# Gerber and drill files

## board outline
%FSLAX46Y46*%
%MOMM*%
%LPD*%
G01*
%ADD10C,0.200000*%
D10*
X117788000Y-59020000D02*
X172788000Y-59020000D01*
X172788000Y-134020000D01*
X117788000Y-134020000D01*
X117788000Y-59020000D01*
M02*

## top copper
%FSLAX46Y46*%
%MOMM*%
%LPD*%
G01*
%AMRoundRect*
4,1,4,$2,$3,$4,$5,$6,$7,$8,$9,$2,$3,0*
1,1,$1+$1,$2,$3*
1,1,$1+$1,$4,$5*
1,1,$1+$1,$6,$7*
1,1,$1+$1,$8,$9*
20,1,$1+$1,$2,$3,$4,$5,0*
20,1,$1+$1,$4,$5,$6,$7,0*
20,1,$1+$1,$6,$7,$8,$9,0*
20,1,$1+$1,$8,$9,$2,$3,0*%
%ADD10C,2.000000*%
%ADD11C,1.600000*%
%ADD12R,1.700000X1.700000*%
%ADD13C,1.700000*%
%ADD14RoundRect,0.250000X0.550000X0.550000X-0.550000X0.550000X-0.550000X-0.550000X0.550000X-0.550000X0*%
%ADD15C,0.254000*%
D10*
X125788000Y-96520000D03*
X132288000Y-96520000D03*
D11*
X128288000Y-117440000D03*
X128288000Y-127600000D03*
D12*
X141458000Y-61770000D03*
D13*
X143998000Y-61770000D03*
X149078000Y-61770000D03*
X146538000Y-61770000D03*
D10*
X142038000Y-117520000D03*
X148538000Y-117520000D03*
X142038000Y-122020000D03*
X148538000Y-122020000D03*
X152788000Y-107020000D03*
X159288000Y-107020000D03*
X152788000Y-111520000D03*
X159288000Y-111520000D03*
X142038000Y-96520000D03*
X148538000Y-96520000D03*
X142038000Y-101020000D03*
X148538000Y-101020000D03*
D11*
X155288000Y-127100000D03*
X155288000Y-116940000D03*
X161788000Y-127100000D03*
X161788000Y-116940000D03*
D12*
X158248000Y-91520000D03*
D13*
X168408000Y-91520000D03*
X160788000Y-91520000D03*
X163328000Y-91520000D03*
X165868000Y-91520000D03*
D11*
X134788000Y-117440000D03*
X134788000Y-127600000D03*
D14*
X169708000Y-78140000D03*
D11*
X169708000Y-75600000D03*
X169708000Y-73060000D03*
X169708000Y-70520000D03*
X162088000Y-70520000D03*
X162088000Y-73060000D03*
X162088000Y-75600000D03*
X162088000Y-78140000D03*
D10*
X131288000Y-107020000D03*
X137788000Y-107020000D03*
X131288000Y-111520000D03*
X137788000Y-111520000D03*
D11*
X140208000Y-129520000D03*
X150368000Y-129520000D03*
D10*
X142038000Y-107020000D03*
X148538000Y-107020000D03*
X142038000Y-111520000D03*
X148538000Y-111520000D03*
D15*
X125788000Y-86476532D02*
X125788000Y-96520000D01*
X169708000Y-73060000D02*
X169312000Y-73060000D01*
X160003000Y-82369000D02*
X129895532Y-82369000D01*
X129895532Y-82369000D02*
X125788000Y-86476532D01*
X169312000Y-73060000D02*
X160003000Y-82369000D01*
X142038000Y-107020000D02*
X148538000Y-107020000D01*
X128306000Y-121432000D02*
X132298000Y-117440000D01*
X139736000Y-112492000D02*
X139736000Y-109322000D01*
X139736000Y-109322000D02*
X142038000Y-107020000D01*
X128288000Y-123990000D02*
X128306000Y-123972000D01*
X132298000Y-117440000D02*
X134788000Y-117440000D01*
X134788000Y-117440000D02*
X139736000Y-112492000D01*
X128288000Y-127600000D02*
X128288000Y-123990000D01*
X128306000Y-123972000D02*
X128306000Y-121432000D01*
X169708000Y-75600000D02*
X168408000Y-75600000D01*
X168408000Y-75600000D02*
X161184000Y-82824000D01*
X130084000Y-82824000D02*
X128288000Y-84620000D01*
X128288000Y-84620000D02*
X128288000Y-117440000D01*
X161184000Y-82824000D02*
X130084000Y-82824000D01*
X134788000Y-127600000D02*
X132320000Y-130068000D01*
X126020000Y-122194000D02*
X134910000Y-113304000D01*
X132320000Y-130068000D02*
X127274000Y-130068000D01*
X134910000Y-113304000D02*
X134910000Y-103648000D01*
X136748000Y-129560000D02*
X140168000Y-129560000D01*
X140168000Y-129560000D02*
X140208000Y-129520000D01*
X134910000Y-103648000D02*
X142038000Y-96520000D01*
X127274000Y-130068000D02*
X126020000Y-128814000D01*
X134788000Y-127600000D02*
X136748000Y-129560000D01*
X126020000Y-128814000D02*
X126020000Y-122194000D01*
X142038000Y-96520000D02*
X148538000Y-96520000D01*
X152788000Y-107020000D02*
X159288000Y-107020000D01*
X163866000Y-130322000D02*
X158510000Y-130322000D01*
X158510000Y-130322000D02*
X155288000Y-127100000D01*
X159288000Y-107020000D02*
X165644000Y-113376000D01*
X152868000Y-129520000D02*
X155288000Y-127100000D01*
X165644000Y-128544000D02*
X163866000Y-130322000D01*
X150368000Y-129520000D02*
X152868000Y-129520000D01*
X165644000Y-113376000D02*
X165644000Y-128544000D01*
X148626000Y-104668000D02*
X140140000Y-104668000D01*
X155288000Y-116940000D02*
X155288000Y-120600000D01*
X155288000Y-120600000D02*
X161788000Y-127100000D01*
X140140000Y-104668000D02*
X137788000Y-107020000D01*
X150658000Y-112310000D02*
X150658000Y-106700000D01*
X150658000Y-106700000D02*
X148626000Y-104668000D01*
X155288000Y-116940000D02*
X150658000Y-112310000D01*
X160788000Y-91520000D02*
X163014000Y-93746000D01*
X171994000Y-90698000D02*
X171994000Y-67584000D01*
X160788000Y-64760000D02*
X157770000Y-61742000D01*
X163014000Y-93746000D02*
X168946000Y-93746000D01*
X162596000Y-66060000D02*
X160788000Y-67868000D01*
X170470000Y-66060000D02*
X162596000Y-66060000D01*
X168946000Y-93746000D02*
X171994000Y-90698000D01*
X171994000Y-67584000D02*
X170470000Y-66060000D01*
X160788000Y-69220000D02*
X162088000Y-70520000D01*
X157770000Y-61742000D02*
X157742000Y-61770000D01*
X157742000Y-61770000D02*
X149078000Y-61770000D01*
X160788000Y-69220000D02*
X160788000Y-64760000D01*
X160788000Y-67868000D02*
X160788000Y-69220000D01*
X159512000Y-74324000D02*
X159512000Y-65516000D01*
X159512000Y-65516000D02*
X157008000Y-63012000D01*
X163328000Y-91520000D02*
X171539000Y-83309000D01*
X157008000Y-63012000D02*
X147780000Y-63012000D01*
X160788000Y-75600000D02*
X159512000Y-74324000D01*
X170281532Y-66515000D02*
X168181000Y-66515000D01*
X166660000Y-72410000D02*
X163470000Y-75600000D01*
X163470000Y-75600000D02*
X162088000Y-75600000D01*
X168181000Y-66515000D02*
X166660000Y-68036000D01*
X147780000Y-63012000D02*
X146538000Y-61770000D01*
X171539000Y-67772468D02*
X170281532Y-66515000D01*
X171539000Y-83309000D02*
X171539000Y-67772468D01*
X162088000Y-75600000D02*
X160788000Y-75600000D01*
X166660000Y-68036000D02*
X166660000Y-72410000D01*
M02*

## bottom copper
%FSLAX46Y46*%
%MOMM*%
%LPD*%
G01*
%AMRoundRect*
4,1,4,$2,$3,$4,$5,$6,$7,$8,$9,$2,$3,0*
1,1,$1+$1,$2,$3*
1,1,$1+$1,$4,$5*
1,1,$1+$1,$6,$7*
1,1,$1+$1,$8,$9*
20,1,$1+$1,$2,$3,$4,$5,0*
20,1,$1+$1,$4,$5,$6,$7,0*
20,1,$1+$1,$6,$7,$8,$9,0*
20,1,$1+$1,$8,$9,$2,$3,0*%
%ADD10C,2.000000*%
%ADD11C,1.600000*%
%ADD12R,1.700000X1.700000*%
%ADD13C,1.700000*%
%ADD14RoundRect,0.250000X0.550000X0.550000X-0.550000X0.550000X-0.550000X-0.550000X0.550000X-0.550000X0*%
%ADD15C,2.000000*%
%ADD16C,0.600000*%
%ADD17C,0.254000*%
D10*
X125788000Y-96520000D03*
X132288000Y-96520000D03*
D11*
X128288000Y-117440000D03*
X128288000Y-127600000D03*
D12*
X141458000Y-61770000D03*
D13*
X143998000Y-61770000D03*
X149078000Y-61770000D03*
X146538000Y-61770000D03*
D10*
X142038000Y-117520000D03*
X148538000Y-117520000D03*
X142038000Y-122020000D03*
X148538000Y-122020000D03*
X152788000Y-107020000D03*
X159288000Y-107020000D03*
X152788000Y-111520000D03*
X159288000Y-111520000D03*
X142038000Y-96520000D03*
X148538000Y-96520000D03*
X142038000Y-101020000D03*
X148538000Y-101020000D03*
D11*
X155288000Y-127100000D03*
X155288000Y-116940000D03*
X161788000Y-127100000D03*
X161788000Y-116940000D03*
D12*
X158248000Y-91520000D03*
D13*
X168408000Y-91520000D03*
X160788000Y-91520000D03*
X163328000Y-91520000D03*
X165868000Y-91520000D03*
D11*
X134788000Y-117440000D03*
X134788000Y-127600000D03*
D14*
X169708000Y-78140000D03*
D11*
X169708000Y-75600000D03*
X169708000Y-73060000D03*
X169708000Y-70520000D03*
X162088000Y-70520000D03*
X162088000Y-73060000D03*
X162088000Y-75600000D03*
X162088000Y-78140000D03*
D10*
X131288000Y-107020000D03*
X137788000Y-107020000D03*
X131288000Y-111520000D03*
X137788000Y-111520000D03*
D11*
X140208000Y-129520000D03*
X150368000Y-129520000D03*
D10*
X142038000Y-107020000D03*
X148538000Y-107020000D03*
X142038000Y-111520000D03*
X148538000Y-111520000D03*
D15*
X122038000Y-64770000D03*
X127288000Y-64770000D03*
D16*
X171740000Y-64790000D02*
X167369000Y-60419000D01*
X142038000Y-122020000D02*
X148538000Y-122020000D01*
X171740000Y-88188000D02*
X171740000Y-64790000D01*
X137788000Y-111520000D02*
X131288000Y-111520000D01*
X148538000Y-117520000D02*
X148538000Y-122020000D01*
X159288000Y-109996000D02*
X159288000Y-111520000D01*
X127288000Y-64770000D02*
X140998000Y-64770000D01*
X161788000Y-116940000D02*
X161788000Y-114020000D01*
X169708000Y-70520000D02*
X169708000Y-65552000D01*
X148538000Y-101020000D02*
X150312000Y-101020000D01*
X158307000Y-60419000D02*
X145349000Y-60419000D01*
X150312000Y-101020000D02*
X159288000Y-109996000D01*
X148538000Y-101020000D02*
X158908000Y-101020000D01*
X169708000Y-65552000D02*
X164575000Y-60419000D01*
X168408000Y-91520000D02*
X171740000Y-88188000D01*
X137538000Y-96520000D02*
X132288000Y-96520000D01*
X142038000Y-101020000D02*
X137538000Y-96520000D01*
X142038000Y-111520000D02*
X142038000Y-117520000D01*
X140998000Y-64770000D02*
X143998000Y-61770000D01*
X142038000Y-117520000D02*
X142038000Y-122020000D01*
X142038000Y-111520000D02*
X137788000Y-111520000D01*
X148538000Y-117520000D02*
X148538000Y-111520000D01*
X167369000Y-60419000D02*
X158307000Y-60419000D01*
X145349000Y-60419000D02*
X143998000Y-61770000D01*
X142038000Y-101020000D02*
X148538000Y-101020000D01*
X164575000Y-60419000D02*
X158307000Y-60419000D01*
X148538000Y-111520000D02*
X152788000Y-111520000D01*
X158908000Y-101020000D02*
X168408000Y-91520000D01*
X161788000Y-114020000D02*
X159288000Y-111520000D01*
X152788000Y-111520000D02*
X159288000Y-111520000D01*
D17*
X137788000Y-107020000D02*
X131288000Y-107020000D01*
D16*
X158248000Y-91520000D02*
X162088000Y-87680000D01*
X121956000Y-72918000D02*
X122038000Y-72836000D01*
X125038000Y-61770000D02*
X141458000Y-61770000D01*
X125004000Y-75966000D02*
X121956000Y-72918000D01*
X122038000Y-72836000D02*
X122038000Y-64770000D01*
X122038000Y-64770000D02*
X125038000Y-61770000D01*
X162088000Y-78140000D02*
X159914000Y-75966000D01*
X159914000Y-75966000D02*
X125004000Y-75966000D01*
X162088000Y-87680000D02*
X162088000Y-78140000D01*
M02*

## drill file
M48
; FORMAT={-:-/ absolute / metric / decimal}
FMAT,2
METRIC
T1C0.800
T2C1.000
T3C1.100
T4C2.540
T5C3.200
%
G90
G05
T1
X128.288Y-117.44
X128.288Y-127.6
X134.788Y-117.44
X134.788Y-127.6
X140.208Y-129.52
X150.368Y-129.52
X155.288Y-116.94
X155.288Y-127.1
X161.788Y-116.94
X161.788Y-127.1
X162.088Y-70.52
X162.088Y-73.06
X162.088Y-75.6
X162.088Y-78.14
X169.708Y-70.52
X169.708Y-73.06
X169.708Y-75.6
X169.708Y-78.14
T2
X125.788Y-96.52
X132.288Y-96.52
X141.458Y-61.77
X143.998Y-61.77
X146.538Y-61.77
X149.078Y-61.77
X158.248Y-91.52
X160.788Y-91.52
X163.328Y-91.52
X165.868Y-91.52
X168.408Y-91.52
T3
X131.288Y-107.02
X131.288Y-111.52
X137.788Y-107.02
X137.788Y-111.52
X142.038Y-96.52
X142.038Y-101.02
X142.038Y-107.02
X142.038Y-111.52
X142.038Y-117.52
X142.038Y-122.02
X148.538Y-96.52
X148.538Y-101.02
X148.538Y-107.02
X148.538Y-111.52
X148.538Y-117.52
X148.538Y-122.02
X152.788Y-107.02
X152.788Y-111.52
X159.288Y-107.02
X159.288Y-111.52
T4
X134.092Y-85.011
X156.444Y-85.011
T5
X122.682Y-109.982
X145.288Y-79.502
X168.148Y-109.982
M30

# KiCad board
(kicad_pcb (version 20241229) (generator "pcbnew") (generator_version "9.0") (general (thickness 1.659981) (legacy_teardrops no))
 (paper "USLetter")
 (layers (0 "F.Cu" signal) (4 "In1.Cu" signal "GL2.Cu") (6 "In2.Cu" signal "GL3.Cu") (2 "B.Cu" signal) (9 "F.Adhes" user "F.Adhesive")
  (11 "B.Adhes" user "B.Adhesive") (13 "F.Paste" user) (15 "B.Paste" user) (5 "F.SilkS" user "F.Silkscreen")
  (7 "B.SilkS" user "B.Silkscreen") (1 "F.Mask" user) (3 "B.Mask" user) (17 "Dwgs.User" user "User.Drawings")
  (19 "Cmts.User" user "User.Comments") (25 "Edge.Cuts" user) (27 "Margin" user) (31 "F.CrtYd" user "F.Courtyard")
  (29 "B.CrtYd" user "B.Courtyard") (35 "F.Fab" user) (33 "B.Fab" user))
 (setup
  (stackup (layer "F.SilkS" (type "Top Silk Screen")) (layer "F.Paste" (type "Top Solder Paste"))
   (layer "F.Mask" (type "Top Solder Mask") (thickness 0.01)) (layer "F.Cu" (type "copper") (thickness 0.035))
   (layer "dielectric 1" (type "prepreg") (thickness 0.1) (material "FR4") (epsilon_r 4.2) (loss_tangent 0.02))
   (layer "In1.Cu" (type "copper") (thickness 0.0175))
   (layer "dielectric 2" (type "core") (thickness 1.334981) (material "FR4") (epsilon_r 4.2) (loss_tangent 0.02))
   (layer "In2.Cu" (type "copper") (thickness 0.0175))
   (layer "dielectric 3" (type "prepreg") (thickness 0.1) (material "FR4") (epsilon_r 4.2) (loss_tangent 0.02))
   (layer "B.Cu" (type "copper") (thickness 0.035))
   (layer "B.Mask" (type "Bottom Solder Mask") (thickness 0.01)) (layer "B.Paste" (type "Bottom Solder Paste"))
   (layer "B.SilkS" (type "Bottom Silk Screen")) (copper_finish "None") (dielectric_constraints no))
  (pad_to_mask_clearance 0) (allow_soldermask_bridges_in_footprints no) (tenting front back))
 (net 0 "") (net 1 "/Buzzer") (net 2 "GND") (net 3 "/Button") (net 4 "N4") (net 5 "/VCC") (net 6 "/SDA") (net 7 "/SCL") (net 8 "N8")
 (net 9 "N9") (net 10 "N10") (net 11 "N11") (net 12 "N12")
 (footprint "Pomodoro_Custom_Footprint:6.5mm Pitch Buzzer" (layer "F.Cu") (at 129.038 96.52)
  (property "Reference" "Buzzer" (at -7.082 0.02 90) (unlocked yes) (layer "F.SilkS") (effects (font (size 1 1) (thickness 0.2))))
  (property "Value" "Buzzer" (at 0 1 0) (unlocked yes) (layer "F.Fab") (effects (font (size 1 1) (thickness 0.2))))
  (pad "1" thru_hole circle (at -3.25 0) (size 2 2) (drill 1) (layers "*.Cu" "*.Mask") (remove_unused_layers no) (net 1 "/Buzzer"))
  (pad "2" thru_hole circle (at 3.25 0) (size 2 2) (drill 1) (layers "*.Cu" "*.Mask") (remove_unused_layers no) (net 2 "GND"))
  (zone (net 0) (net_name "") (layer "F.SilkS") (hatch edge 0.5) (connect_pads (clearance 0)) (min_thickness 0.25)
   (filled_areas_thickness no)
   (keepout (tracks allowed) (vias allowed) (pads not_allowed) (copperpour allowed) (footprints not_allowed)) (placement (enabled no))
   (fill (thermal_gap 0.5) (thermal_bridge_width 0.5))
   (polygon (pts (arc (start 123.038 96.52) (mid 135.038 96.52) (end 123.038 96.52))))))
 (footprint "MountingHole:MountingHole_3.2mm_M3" (layer "F.Cu") (at 168.148 109.982)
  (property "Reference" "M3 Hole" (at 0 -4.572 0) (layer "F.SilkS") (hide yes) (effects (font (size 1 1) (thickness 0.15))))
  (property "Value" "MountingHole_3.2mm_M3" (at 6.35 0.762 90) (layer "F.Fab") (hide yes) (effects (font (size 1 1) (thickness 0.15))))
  (pad "" np_thru_hole circle (at 0 0) (size 3.2 3.2) (drill 3.2) (layers "*.Cu" "*.Mask")))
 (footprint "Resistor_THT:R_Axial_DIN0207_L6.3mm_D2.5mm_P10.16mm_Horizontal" (layer "F.Cu") (at 128.288 117.44 -90)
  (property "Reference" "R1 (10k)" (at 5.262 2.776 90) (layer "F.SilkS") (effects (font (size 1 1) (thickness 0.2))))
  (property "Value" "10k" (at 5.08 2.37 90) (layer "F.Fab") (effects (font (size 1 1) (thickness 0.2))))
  (pad "1" thru_hole circle (at 0 0 270) (size 1.6 1.6) (drill 0.8) (layers "*.Cu" "*.Mask") (remove_unused_layers no) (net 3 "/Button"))
  (pad "2" thru_hole circle (at 10.16 0 270) (size 1.6 1.6) (drill 0.8) (layers "*.Cu" "*.Mask") (remove_unused_layers no) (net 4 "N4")))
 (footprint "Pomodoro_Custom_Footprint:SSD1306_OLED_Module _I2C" (layer "F.Cu") (at 145.268 73.835)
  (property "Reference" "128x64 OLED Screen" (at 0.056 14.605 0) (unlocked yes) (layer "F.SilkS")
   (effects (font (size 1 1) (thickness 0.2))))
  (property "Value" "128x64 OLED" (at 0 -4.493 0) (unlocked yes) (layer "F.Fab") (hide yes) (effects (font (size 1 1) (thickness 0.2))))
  (pad "" np_thru_hole circle (at -11.176 11.176) (size 1.7 1.7) (drill 2.54) (layers "*.Cu" "*.Mask"))
  (pad "" np_thru_hole circle (at 11.176 11.176) (size 1.7 1.7) (drill 2.54) (layers "*.Cu" "*.Mask"))
  (pad "1" thru_hole rect (at -3.81 -12.065) (size 1.7 1.7) (drill 1) (layers "*.Cu" "*.Mask") (remove_unused_layers no) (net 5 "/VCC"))
  (pad "2" thru_hole circle (at -1.27 -12.065) (size 1.7 1.7) (drill 1) (layers "*.Cu" "*.Mask") (remove_unused_layers no) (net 2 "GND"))
  (pad "3" thru_hole circle (at 3.81 -12.065) (size 1.7 1.7) (drill 1) (layers "*.Cu" "*.Mask") (remove_unused_layers no) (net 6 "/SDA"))
  (pad "4" thru_hole circle (at 1.27 -12.065) (size 1.7 1.7) (drill 1) (layers "*.Cu" "*.Mask") (remove_unused_layers no) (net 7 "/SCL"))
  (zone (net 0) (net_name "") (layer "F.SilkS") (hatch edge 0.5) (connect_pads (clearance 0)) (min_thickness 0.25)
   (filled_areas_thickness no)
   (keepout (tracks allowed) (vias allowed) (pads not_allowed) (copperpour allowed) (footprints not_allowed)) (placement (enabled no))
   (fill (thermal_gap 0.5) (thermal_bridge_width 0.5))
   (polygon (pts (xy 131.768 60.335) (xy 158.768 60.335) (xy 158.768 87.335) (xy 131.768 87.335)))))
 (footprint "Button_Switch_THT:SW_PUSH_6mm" (layer "F.Cu") (at 142.038 117.52)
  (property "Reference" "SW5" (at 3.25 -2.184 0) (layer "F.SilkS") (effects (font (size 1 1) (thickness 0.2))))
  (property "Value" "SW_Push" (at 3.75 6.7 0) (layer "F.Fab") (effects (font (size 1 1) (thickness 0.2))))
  (pad "1" thru_hole circle (at 0 0 90) (size 2 2) (drill 1.1) (layers "*.Cu" "*.Mask") (remove_unused_layers no) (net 2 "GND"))
  (pad "1" thru_hole circle (at 6.5 0 90) (size 2 2) (drill 1.1) (layers "*.Cu" "*.Mask") (remove_unused_layers no) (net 2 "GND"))
  (pad "2" thru_hole circle (at 0 4.5 90) (size 2 2) (drill 1.1) (layers "*.Cu" "*.Mask") (remove_unused_layers no) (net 2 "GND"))
  (pad "2" thru_hole circle (at 6.5 4.5 90) (size 2 2) (drill 1.1) (layers "*.Cu" "*.Mask") (remove_unused_layers no) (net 2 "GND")))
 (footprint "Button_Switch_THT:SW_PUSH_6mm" (layer "F.Cu") (at 152.788 107.02)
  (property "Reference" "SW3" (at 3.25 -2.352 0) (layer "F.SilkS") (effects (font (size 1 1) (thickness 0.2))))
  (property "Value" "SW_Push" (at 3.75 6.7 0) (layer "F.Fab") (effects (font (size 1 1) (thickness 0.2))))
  (pad "1" thru_hole circle (at 0 0 90) (size 2 2) (drill 1.1) (layers "*.Cu" "*.Mask") (remove_unused_layers no) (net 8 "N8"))
  (pad "1" thru_hole circle (at 6.5 0 90) (size 2 2) (drill 1.1) (layers "*.Cu" "*.Mask") (remove_unused_layers no) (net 8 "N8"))
  (pad "2" thru_hole circle (at 0 4.5 90) (size 2 2) (drill 1.1) (layers "*.Cu" "*.Mask") (remove_unused_layers no) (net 2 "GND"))
  (pad "2" thru_hole circle (at 6.5 4.5 90) (size 2 2) (drill 1.1) (layers "*.Cu" "*.Mask") (remove_unused_layers no) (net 2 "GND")))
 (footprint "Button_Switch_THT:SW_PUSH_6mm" (layer "F.Cu") (at 142.038 96.52)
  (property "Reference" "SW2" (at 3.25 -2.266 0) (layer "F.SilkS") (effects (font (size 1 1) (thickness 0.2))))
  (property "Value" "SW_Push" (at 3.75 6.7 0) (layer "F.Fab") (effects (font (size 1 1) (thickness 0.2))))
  (pad "1" thru_hole circle (at 0 0 90) (size 2 2) (drill 1.1) (layers "*.Cu" "*.Mask") (remove_unused_layers no) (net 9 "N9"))
  (pad "1" thru_hole circle (at 6.5 0 90) (size 2 2) (drill 1.1) (layers "*.Cu" "*.Mask") (remove_unused_layers no) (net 9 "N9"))
  (pad "2" thru_hole circle (at 0 4.5 90) (size 2 2) (drill 1.1) (layers "*.Cu" "*.Mask") (remove_unused_layers no) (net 2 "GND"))
  (pad "2" thru_hole circle (at 6.5 4.5 90) (size 2 2) (drill 1.1) (layers "*.Cu" "*.Mask") (remove_unused_layers no) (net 2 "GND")))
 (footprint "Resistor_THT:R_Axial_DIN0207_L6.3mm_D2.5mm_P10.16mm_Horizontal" (layer "F.Cu") (at 155.288 127.1 90)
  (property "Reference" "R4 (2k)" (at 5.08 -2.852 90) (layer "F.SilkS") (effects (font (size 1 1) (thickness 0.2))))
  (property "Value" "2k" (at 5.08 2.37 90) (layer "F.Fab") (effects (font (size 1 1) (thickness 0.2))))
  (pad "1" thru_hole circle (at 0 0 90) (size 1.6 1.6) (drill 0.8) (layers "*.Cu" "*.Mask") (remove_unused_layers no) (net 8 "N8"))
  (pad "2" thru_hole circle (at 10.16 0 90) (size 1.6 1.6) (drill 0.8) (layers "*.Cu" "*.Mask") (remove_unused_layers no) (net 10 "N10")))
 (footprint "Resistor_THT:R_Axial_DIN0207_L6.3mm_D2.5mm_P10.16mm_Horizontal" (layer "F.Cu") (at 161.788 127.1 90)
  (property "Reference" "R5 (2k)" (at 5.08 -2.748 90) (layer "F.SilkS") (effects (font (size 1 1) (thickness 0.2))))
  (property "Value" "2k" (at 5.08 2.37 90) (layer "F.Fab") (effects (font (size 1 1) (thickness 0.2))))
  (pad "1" thru_hole circle (at 0 0 90) (size 1.6 1.6) (drill 0.8) (layers "*.Cu" "*.Mask") (remove_unused_layers no) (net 10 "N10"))
  (pad "2" thru_hole circle (at 10.16 0 90) (size 1.6 1.6) (drill 0.8) (layers "*.Cu" "*.Mask") (remove_unused_layers no) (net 2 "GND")))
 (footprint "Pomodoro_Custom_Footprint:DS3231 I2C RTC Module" (layer "F.Cu") (at 163.328 96.6)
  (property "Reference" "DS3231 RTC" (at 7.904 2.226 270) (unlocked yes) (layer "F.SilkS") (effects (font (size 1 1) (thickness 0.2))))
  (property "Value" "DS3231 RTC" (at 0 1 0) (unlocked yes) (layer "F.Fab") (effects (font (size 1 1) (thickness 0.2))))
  (pad "1" thru_hole rect (at -5.08 -5.08) (size 1.7 1.7) (drill 1) (layers "*.Cu" "*.Mask") (remove_unused_layers no) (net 5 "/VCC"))
  (pad "2" thru_hole circle (at 5.08 -5.08) (size 1.7 1.7) (drill 1) (layers "*.Cu" "*.Mask") (remove_unused_layers no) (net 2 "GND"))
  (pad "3" thru_hole circle (at -2.54 -5.08) (size 1.7 1.7) (drill 1) (layers "*.Cu" "*.Mask") (remove_unused_layers no) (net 6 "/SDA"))
  (pad "4" thru_hole circle (at 0 -5.08) (size 1.7 1.7) (drill 1) (layers "*.Cu" "*.Mask") (remove_unused_layers no) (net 7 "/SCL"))
  (pad "5" thru_hole circle (at 2.54 -5.08) (size 1.7 1.7) (drill 1) (layers "*.Cu" "*.Mask") (remove_unused_layers no))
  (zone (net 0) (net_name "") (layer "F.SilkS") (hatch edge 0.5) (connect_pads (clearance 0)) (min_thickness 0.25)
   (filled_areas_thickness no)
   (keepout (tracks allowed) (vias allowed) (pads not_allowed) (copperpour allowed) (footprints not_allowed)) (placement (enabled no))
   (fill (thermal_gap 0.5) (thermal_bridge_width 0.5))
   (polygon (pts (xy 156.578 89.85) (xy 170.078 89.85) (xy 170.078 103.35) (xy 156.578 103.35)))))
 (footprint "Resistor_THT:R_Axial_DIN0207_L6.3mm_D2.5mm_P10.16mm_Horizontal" (layer "F.Cu") (at 134.788 117.44 -90)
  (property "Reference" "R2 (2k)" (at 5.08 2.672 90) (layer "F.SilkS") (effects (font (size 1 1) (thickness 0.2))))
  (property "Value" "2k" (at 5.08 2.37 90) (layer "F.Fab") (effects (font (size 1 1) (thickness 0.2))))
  (pad "1" thru_hole circle (at 0 0 270) (size 1.6 1.6) (drill 0.8) (layers "*.Cu" "*.Mask") (remove_unused_layers no) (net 4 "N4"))
  (pad "2" thru_hole circle (at 10.16 0 270) (size 1.6 1.6) (drill 0.8) (layers "*.Cu" "*.Mask") (remove_unused_layers no) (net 9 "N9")))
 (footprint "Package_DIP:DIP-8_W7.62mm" (layer "F.Cu") (at 169.708 78.14 180)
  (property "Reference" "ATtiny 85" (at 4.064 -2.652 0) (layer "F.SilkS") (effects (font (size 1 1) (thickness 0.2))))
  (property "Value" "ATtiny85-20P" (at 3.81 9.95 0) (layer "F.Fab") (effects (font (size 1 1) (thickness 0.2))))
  (pad "1" thru_hole roundrect (at 0 0 180) (size 1.6 1.6) (drill 0.8) (layers "*.Cu" "*.Mask") (remove_unused_layers no)
   (roundrect_rratio 0.15625) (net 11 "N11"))
  (pad "2" thru_hole circle (at 0 2.54 180) (size 1.6 1.6) (drill 0.8) (layers "*.Cu" "*.Mask") (remove_unused_layers no) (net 3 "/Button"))
  (pad "3" thru_hole circle (at 0 5.08 180) (size 1.6 1.6) (drill 0.8) (layers "*.Cu" "*.Mask") (remove_unused_layers no) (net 1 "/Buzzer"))
  (pad "4" thru_hole circle (at 0 7.62 180) (size 1.6 1.6) (drill 0.8) (layers "*.Cu" "*.Mask") (remove_unused_layers no) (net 2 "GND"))
  (pad "5" thru_hole circle (at 7.62 7.62 180) (size 1.6 1.6) (drill 0.8) (layers "*.Cu" "*.Mask") (remove_unused_layers no) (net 6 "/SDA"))
  (pad "6" thru_hole circle (at 7.62 5.08 180) (size 1.6 1.6) (drill 0.8) (layers "*.Cu" "*.Mask") (remove_unused_layers no) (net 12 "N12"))
  (pad "7" thru_hole circle (at 7.62 2.54 180) (size 1.6 1.6) (drill 0.8) (layers "*.Cu" "*.Mask") (remove_unused_layers no) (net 7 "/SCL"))
  (pad "8" thru_hole circle (at 7.62 0 180) (size 1.6 1.6) (drill 0.8) (layers "*.Cu" "*.Mask") (remove_unused_layers no) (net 5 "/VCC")))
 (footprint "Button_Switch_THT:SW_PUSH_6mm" (layer "F.Cu") (at 131.288 107.02)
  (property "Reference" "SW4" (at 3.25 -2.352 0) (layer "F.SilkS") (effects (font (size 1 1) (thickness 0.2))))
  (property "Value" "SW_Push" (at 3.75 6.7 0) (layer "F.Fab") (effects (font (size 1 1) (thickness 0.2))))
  (pad "1" thru_hole circle (at 0 0 90) (size 2 2) (drill 1.1) (layers "*.Cu" "*.Mask") (remove_unused_layers no) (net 10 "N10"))
  (pad "1" thru_hole circle (at 6.5 0 90) (size 2 2) (drill 1.1) (layers "*.Cu" "*.Mask") (remove_unused_layers no) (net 10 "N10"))
  (pad "2" thru_hole circle (at 0 4.5 90) (size 2 2) (drill 1.1) (layers "*.Cu" "*.Mask") (remove_unused_layers no) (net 2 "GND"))
  (pad "2" thru_hole circle (at 6.5 4.5 90) (size 2 2) (drill 1.1) (layers "*.Cu" "*.Mask") (remove_unused_layers no) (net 2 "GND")))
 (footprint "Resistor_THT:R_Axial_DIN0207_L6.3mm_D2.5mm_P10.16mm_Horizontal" (layer "F.Cu") (at 140.208 129.52)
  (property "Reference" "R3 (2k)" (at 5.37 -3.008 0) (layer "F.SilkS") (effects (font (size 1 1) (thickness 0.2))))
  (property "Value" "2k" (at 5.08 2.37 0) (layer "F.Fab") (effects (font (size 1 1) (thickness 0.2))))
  (pad "1" thru_hole circle (at 0 0) (size 1.6 1.6) (drill 0.8) (layers "*.Cu" "*.Mask") (remove_unused_layers no) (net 9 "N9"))
  (pad "2" thru_hole circle (at 10.16 0) (size 1.6 1.6) (drill 0.8) (layers "*.Cu" "*.Mask") (remove_unused_layers no) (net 8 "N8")))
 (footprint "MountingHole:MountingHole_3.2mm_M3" (layer "F.Cu") (at 145.288 79.502)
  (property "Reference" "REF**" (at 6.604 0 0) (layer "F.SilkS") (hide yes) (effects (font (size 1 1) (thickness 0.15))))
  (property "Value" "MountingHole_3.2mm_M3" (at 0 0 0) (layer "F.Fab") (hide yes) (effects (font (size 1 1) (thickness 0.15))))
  (pad "" np_thru_hole circle (at 0 0) (size 3.2 3.2) (drill 3.2) (layers "*.Cu" "*.Mask")))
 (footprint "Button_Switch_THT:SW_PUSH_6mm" (layer "F.Cu") (at 142.038 107.02)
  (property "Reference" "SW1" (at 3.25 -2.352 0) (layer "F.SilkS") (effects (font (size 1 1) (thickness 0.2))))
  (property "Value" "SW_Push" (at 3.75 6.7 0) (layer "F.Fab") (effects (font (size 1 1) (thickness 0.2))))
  (pad "1" thru_hole circle (at 0 0 90) (size 2 2) (drill 1.1) (layers "*.Cu" "*.Mask") (remove_unused_layers no) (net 4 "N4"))
  (pad "1" thru_hole circle (at 6.5 0 90) (size 2 2) (drill 1.1) (layers "*.Cu" "*.Mask") (remove_unused_layers no) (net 4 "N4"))
  (pad "2" thru_hole circle (at 0 4.5 90) (size 2 2) (drill 1.1) (layers "*.Cu" "*.Mask") (remove_unused_layers no) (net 2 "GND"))
  (pad "2" thru_hole circle (at 6.5 4.5 90) (size 2 2) (drill 1.1) (layers "*.Cu" "*.Mask") (remove_unused_layers no) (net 2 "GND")))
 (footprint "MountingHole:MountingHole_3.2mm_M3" (layer "F.Cu") (at 122.682 109.982)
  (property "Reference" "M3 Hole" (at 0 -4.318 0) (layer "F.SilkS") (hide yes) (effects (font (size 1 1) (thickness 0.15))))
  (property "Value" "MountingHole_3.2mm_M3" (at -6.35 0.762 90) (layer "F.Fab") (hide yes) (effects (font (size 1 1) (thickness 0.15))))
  (pad "" np_thru_hole circle (at 0 0) (size 3.2 3.2) (drill 3.2) (layers "*.Cu" "*.Mask")))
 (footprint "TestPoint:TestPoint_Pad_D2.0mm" (layer "B.Cu") (at 122.038 64.77 180)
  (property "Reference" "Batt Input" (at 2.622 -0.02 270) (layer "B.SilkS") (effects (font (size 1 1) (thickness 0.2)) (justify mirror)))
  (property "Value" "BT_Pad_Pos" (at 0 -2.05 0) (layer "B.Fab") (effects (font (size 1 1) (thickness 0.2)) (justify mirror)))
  (pad "1" smd circle (at 0 0 180) (size 2 2) (layers "B.Cu" "B.Mask") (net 5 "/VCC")))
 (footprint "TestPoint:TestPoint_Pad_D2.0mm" (layer "B.Cu") (at 127.288 64.77 180)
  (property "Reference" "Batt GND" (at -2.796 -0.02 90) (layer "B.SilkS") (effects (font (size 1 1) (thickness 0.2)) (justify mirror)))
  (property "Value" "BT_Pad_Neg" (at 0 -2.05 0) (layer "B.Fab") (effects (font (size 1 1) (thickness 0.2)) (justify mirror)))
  (pad "1" smd circle (at 0 0 180) (size 2 2) (layers "B.Cu" "B.Mask") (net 2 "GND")))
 (gr_rect (start 117.788 59.02) (end 172.788 134.02) (stroke (width 0.2) (type default)) (fill no) (layer "Edge.Cuts"))
 (segment (start 125.788 86.476532) (end 125.788 96.52) (width 0.254) (layer "F.Cu") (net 1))
 (segment (start 169.708 73.06) (end 169.312 73.06) (width 0.254) (layer "F.Cu") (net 1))
 (segment (start 160.003 82.369) (end 129.895532 82.369) (width 0.254) (layer "F.Cu") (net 1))
 (segment (start 129.895532 82.369) (end 125.788 86.476532) (width 0.254) (layer "F.Cu") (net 1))
 (segment (start 169.312 73.06) (end 160.003 82.369) (width 0.254) (layer "F.Cu") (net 1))
 (segment (start 171.74 64.79) (end 167.369 60.419) (width 0.6) (layer "B.Cu") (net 2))
 (segment (start 142.038 122.02) (end 148.538 122.02) (width 0.6) (layer "B.Cu") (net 2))
 (segment (start 171.74 88.188) (end 171.74 64.79) (width 0.6) (layer "B.Cu") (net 2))
 (segment (start 137.788 111.52) (end 131.288 111.52) (width 0.6) (layer "B.Cu") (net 2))
 (segment (start 148.538 117.52) (end 148.538 122.02) (width 0.6) (layer "B.Cu") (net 2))
 (segment (start 159.288 109.996) (end 159.288 111.52) (width 0.6) (layer "B.Cu") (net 2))
 (segment (start 127.288 64.77) (end 140.998 64.77) (width 0.6) (layer "B.Cu") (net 2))
 (segment (start 161.788 116.94) (end 161.788 114.02) (width 0.6) (layer "B.Cu") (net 2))
 (segment (start 169.708 70.52) (end 169.708 65.552) (width 0.6) (layer "B.Cu") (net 2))
 (segment (start 148.538 101.02) (end 150.312 101.02) (width 0.6) (layer "B.Cu") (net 2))
 (segment (start 158.307 60.419) (end 145.349 60.419) (width 0.6) (layer "B.Cu") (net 2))
 (segment (start 150.312 101.02) (end 159.288 109.996) (width 0.6) (layer "B.Cu") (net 2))
 (segment (start 148.538 101.02) (end 158.908 101.02) (width 0.6) (layer "B.Cu") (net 2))
 (segment (start 169.708 65.552) (end 164.575 60.419) (width 0.6) (layer "B.Cu") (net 2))
 (segment (start 168.408 91.52) (end 171.74 88.188) (width 0.6) (layer "B.Cu") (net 2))
 (segment (start 137.538 96.52) (end 132.288 96.52) (width 0.6) (layer "B.Cu") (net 2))
 (segment (start 142.038 101.02) (end 137.538 96.52) (width 0.6) (layer "B.Cu") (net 2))
 (segment (start 142.038 111.52) (end 142.038 117.52) (width 0.6) (layer "B.Cu") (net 2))
 (segment (start 140.998 64.77) (end 143.998 61.77) (width 0.6) (layer "B.Cu") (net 2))
 (segment (start 142.038 117.52) (end 142.038 122.02) (width 0.6) (layer "B.Cu") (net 2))
 (segment (start 142.038 111.52) (end 137.788 111.52) (width 0.6) (layer "B.Cu") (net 2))
 (segment (start 148.538 117.52) (end 148.538 111.52) (width 0.6) (layer "B.Cu") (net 2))
 (segment (start 167.369 60.419) (end 158.307 60.419) (width 0.6) (layer "B.Cu") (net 2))
 (segment (start 145.349 60.419) (end 143.998 61.77) (width 0.6) (layer "B.Cu") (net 2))
 (segment (start 142.038 101.02) (end 148.538 101.02) (width 0.6) (layer "B.Cu") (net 2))
 (segment (start 164.575 60.419) (end 158.307 60.419) (width 0.6) (layer "B.Cu") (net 2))
 (segment (start 148.538 111.52) (end 152.788 111.52) (width 0.6) (layer "B.Cu") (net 2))
 (segment (start 158.908 101.02) (end 168.408 91.52) (width 0.6) (layer "B.Cu") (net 2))
 (segment (start 161.788 114.02) (end 159.288 111.52) (width 0.6) (layer "B.Cu") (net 2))
 (segment (start 152.788 111.52) (end 159.288 111.52) (width 0.6) (layer "B.Cu") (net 2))
 (segment (start 142.038 107.02) (end 148.538 107.02) (width 0.254) (layer "F.Cu") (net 4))
 (segment (start 128.306 121.432) (end 132.298 117.44) (width 0.254) (layer "F.Cu") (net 4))
 (segment (start 139.736 112.492) (end 139.736 109.322) (width 0.254) (layer "F.Cu") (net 4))
 (segment (start 139.736 109.322) (end 142.038 107.02) (width 0.254) (layer "F.Cu") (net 4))
 (segment (start 128.288 123.99) (end 128.306 123.972) (width 0.254) (layer "F.Cu") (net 4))
 (segment (start 132.298 117.44) (end 134.788 117.44) (width 0.254) (layer "F.Cu") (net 4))
 (segment (start 134.788 117.44) (end 139.736 112.492) (width 0.254) (layer "F.Cu") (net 4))
 (segment (start 128.288 127.6) (end 128.288 123.99) (width 0.254) (layer "F.Cu") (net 4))
 (segment (start 128.306 123.972) (end 128.306 121.432) (width 0.254) (layer "F.Cu") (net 4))
 (segment (start 169.708 75.6) (end 168.408 75.6) (width 0.254) (layer "F.Cu") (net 3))
 (segment (start 168.408 75.6) (end 161.184 82.824) (width 0.254) (layer "F.Cu") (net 3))
 (segment (start 130.084 82.824) (end 128.288 84.62) (width 0.254) (layer "F.Cu") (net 3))
 (segment (start 128.288 84.62) (end 128.288 117.44) (width 0.254) (layer "F.Cu") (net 3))
 (segment (start 161.184 82.824) (end 130.084 82.824) (width 0.254) (layer "F.Cu") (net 3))
 (segment (start 134.788 127.6) (end 132.32 130.068) (width 0.254) (layer "F.Cu") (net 9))
 (segment (start 126.02 122.194) (end 134.91 113.304) (width 0.254) (layer "F.Cu") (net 9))
 (segment (start 132.32 130.068) (end 127.274 130.068) (width 0.254) (layer "F.Cu") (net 9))
 (segment (start 134.91 113.304) (end 134.91 103.648) (width 0.254) (layer "F.Cu") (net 9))
 (segment (start 136.748 129.56) (end 140.168 129.56) (width 0.254) (layer "F.Cu") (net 9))
 (segment (start 140.168 129.56) (end 140.208 129.52) (width 0.254) (layer "F.Cu") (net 9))
 (segment (start 134.91 103.648) (end 142.038 96.52) (width 0.254) (layer "F.Cu") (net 9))
 (segment (start 127.274 130.068) (end 126.02 128.814) (width 0.254) (layer "F.Cu") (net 9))
 (segment (start 134.788 127.6) (end 136.748 129.56) (width 0.254) (layer "F.Cu") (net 9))
 (segment (start 126.02 128.814) (end 126.02 122.194) (width 0.254) (layer "F.Cu") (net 9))
 (segment (start 142.038 96.52) (end 148.538 96.52) (width 0.254) (layer "F.Cu") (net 9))
 (segment (start 152.788 107.02) (end 159.288 107.02) (width 0.254) (layer "F.Cu") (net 8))
 (segment (start 163.866 130.322) (end 158.51 130.322) (width 0.254) (layer "F.Cu") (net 8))
 (segment (start 158.51 130.322) (end 155.288 127.1) (width 0.254) (layer "F.Cu") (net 8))
 (segment (start 159.288 107.02) (end 165.644 113.376) (width 0.254) (layer "F.Cu") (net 8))
 (segment (start 152.868 129.52) (end 155.288 127.1) (width 0.254) (layer "F.Cu") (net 8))
 (segment (start 165.644 128.544) (end 163.866 130.322) (width 0.254) (layer "F.Cu") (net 8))
 (segment (start 150.368 129.52) (end 152.868 129.52) (width 0.254) (layer "F.Cu") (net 8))
 (segment (start 165.644 113.376) (end 165.644 128.544) (width 0.254) (layer "F.Cu") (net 8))
 (segment (start 148.626 104.668) (end 140.14 104.668) (width 0.254) (layer "F.Cu") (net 10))
 (segment (start 155.288 116.94) (end 155.288 120.6) (width 0.254) (layer "F.Cu") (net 10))
 (segment (start 155.288 120.6) (end 161.788 127.1) (width 0.254) (layer "F.Cu") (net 10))
 (segment (start 140.14 104.668) (end 137.788 107.02) (width 0.254) (layer "F.Cu") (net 10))
 (segment (start 150.658 112.31) (end 150.658 106.7) (width 0.254) (layer "F.Cu") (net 10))
 (segment (start 150.658 106.7) (end 148.626 104.668) (width 0.254) (layer "F.Cu") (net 10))
 (segment (start 155.288 116.94) (end 150.658 112.31) (width 0.254) (layer "F.Cu") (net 10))
 (segment (start 137.788 107.02) (end 131.288 107.02) (width 0.254) (layer "B.Cu") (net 10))
 (segment (start 158.248 91.52) (end 162.088 87.68) (width 0.6) (layer "B.Cu") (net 5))
 (segment (start 121.956 72.918) (end 122.038 72.836) (width 0.6) (layer "B.Cu") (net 5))
 (segment (start 125.038 61.77) (end 141.458 61.77) (width 0.6) (layer "B.Cu") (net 5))
 (segment (start 125.004 75.966) (end 121.956 72.918) (width 0.6) (layer "B.Cu") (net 5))
 (segment (start 122.038 72.836) (end 122.038 64.77) (width 0.6) (layer "B.Cu") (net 5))
 (segment (start 122.038 64.77) (end 125.038 61.77) (width 0.6) (layer "B.Cu") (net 5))
 (segment (start 162.088 78.14) (end 159.914 75.966) (width 0.6) (layer "B.Cu") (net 5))
 (segment (start 159.914 75.966) (end 125.004 75.966) (width 0.6) (layer "B.Cu") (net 5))
 (segment (start 162.088 87.68) (end 162.088 78.14) (width 0.6) (layer "B.Cu") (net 5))
 (segment (start 160.788 91.52) (end 163.014 93.746) (width 0.254) (layer "F.Cu") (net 6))
 (segment (start 171.994 90.698) (end 171.994 67.584) (width 0.254) (layer "F.Cu") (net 6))
 (segment (start 160.788 64.76) (end 157.77 61.742) (width 0.254) (layer "F.Cu") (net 6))
 (segment (start 163.014 93.746) (end 168.946 93.746) (width 0.254) (layer "F.Cu") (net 6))
 (segment (start 162.596 66.06) (end 160.788 67.868) (width 0.254) (layer "F.Cu") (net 6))
 (segment (start 170.47 66.06) (end 162.596 66.06) (width 0.254) (layer "F.Cu") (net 6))
 (segment (start 168.946 93.746) (end 171.994 90.698) (width 0.254) (layer "F.Cu") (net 6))
 (segment (start 171.994 67.584) (end 170.47 66.06) (width 0.254) (layer "F.Cu") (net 6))
 (segment (start 160.788 69.22) (end 162.088 70.52) (width 0.254) (layer "F.Cu") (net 6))
 (segment (start 157.77 61.742) (end 157.742 61.77) (width 0.254) (layer "F.Cu") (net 6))
 (segment (start 157.742 61.77) (end 149.078 61.77) (width 0.254) (layer "F.Cu") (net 6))
 (segment (start 160.788 69.22) (end 160.788 64.76) (width 0.254) (layer "F.Cu") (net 6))
 (segment (start 160.788 67.868) (end 160.788 69.22) (width 0.254) (layer "F.Cu") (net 6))
 (segment (start 159.512 74.324) (end 159.512 65.516) (width 0.254) (layer "F.Cu") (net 7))
 (segment (start 159.512 65.516) (end 157.008 63.012) (width 0.254) (layer "F.Cu") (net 7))
 (segment (start 163.328 91.52) (end 171.539 83.309) (width 0.254) (layer "F.Cu") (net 7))
 (segment (start 157.008 63.012) (end 147.78 63.012) (width 0.254) (layer "F.Cu") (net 7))
 (segment (start 160.788 75.6) (end 159.512 74.324) (width 0.254) (layer "F.Cu") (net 7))
 (segment (start 170.281532 66.515) (end 168.181 66.515) (width 0.254) (layer "F.Cu") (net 7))
 (segment (start 166.66 72.41) (end 163.47 75.6) (width 0.254) (layer "F.Cu") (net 7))
 (segment (start 163.47 75.6) (end 162.088 75.6) (width 0.254) (layer "F.Cu") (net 7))
 (segment (start 168.181 66.515) (end 166.66 68.036) (width 0.254) (layer "F.Cu") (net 7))
 (segment (start 147.78 63.012) (end 146.538 61.77) (width 0.254) (layer "F.Cu") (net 7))
 (segment (start 171.539 67.772468) (end 170.281532 66.515) (width 0.254) (layer "F.Cu") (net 7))
 (segment (start 171.539 83.309) (end 171.539 67.772468) (width 0.254) (layer "F.Cu") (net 7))
 (segment (start 162.088 75.6) (end 160.788 75.6) (width 0.254) (layer "F.Cu") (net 7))
 (segment (start 166.66 68.036) (end 166.66 72.41) (width 0.254) (layer "F.Cu") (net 7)))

